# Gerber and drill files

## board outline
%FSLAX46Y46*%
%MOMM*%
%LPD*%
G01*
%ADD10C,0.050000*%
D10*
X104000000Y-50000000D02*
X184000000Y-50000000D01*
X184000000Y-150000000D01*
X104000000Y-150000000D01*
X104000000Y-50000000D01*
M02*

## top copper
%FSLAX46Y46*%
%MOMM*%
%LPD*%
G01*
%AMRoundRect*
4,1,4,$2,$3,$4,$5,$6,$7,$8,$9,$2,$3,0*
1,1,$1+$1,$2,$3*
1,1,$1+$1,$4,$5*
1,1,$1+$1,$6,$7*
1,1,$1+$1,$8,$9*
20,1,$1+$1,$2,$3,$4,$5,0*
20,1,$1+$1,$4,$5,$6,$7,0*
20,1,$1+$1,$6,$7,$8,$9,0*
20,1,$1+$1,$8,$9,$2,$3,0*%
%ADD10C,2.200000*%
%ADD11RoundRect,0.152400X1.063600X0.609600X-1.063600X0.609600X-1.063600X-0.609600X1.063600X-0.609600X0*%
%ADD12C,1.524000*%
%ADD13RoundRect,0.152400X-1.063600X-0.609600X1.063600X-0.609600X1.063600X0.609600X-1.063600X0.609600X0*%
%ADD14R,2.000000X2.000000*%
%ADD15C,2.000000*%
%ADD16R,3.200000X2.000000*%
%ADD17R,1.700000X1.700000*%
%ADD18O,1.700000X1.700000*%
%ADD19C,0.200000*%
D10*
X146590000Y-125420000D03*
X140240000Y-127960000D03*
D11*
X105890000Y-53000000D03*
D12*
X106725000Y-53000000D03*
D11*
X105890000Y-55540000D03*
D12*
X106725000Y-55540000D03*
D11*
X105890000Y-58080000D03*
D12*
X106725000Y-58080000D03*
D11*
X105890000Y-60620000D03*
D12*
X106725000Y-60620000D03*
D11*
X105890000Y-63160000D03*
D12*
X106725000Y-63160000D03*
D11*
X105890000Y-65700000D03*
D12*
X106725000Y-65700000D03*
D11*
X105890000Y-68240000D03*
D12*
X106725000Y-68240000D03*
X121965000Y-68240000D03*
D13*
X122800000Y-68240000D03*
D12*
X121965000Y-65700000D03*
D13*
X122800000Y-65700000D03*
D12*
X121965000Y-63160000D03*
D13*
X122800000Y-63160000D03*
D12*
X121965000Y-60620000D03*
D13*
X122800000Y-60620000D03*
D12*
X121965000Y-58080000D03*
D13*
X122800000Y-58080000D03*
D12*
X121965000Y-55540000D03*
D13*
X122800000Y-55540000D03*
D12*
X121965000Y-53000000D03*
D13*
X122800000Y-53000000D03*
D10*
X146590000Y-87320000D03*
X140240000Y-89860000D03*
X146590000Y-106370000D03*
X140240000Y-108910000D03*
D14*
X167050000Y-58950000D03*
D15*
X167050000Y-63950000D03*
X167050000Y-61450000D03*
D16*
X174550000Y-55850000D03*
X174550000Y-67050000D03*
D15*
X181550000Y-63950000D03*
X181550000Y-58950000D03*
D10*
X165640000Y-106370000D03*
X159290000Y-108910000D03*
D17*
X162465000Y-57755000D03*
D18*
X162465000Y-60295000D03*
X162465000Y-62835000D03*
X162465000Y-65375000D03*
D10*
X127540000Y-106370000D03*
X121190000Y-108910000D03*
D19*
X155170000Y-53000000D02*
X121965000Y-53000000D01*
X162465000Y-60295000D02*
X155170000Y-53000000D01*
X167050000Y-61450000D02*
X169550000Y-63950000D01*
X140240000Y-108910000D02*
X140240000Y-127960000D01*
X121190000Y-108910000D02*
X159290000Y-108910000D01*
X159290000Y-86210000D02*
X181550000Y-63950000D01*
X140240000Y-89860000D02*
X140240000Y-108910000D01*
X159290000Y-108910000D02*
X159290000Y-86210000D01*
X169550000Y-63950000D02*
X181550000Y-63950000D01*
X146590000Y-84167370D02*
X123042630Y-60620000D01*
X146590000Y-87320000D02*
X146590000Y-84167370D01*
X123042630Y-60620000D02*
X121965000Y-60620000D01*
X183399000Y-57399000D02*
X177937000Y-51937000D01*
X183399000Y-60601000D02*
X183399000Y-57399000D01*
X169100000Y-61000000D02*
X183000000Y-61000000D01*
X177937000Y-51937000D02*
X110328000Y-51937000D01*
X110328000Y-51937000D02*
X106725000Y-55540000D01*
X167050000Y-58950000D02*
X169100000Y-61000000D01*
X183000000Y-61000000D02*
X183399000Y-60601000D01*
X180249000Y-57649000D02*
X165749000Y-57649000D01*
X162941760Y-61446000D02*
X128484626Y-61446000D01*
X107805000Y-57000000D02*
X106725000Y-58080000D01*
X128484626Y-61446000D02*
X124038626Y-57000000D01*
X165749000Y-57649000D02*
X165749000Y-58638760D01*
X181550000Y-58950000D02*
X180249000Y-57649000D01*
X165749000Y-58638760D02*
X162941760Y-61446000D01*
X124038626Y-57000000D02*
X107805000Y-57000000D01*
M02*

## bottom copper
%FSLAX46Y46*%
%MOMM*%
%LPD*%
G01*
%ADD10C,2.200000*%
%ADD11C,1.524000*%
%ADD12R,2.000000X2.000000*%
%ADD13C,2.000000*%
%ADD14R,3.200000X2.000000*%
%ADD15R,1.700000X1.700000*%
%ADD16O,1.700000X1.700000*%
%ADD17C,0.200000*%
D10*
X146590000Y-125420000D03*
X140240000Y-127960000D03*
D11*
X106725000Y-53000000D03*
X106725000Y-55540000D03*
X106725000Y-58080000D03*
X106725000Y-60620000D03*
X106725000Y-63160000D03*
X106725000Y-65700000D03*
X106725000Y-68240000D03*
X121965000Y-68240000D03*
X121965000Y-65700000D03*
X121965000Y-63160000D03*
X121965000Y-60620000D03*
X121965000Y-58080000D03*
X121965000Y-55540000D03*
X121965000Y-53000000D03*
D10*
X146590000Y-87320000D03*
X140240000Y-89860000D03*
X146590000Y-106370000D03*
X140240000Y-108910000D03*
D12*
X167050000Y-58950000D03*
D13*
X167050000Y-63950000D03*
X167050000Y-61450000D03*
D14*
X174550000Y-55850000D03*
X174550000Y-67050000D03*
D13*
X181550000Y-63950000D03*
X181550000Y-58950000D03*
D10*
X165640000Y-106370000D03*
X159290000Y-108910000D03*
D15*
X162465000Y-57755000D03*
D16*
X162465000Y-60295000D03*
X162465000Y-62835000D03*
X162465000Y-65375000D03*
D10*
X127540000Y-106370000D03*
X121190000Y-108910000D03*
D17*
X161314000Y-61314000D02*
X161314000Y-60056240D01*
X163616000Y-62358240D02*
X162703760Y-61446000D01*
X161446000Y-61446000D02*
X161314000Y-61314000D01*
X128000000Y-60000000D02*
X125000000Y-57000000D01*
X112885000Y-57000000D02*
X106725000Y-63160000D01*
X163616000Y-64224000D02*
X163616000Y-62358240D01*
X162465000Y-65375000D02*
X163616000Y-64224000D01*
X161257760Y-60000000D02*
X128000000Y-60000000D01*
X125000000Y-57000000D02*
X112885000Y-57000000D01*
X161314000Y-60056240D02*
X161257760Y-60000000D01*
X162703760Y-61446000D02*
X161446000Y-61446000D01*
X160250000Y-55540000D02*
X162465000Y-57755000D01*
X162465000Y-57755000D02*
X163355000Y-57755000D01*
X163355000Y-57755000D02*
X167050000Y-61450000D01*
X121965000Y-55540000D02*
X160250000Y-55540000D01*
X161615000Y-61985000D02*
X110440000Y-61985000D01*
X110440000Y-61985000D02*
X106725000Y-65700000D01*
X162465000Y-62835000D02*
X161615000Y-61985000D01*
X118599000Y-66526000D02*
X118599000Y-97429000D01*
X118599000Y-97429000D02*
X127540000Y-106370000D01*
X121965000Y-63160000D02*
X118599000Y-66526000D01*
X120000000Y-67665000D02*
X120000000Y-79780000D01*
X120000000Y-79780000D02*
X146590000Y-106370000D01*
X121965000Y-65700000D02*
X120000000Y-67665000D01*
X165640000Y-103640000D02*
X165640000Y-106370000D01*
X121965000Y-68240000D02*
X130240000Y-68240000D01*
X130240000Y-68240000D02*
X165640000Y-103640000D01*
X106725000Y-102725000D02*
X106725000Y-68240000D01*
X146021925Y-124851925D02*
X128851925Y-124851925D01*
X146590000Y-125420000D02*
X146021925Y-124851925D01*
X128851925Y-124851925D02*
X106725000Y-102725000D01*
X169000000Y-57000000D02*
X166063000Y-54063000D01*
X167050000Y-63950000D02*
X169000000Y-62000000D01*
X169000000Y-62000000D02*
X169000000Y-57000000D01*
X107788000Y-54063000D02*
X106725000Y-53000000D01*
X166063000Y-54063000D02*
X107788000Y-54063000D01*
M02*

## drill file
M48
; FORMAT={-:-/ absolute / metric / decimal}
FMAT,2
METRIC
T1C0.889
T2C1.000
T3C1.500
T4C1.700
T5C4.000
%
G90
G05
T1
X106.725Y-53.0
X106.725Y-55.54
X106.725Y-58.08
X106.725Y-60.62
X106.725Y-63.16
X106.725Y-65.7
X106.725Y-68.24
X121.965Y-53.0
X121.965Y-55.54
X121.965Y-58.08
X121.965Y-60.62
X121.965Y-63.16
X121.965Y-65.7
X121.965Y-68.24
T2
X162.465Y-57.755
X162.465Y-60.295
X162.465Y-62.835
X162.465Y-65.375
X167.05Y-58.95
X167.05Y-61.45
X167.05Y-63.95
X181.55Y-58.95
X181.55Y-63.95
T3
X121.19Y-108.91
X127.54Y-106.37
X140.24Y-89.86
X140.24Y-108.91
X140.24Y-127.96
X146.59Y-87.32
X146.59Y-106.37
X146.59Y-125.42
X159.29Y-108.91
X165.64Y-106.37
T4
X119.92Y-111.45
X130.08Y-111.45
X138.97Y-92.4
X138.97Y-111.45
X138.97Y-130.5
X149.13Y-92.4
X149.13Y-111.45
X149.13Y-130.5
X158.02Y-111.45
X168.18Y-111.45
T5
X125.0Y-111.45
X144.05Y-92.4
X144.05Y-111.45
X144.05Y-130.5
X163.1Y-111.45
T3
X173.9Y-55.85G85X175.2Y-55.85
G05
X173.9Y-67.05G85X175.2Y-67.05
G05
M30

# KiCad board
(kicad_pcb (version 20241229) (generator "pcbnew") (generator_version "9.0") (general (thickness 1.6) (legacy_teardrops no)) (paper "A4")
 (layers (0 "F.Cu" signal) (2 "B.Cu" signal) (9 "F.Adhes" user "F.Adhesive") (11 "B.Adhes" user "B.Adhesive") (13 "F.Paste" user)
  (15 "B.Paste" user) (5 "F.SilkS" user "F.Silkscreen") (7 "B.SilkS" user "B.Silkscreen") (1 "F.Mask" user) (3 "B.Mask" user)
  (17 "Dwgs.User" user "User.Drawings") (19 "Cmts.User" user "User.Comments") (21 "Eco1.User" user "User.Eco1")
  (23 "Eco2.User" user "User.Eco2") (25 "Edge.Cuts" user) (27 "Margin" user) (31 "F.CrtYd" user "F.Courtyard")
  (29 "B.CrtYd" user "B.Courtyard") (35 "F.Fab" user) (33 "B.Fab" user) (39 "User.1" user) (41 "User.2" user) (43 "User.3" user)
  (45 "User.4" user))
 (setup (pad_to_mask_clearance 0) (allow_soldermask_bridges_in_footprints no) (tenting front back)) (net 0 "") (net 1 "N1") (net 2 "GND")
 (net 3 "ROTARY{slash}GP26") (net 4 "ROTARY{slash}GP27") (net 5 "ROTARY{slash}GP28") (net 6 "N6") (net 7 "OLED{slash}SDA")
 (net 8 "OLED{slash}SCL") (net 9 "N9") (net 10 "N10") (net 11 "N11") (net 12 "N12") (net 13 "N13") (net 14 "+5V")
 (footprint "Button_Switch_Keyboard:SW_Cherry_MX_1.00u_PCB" (layer "F.Cu") (at 146.59 125.42)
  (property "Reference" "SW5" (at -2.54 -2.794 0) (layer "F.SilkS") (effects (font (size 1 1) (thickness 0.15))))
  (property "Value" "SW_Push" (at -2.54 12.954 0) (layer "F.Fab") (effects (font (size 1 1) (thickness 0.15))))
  (pad "" np_thru_hole circle (at -7.62 5.08) (size 1.7 1.7) (drill 1.7) (layers "*.Cu" "*.Mask"))
  (pad "" np_thru_hole circle (at -2.54 5.08) (size 4 4) (drill 4) (layers "*.Cu" "*.Mask"))
  (pad "" np_thru_hole circle (at 2.54 5.08) (size 1.7 1.7) (drill 1.7) (layers "*.Cu" "*.Mask"))
  (pad "1" thru_hole circle (at 0 0) (size 2.2 2.2) (drill 1.5) (layers "*.Cu" "*.Mask") (remove_unused_layers no) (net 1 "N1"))
  (pad "2" thru_hole circle (at -6.35 2.54) (size 2.2 2.2) (drill 1.5) (layers "*.Cu" "*.Mask") (remove_unused_layers no) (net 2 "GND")))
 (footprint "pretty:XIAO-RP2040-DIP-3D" (layer "F.Cu") (at 114.345 60.62)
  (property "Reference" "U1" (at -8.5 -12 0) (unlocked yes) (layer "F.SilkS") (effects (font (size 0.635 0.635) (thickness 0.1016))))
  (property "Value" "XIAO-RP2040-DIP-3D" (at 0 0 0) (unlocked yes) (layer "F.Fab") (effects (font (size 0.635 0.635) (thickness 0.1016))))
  (pad "1" smd roundrect (at -8.455 -7.62 180) (size 2.432 1.524) (layers "F.Cu" "F.Mask") (roundrect_rratio 0.1)
   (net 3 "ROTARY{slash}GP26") (thermal_bridge_angle 45))
  (pad "1" thru_hole circle (at -7.62 -7.62 180) (size 1.524 1.524) (drill 0.889) (layers "*.Cu" "*.Mask") (remove_unused_layers no)
   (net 3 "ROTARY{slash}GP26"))
  (pad "2" smd roundrect (at -8.455 -5.08 180) (size 2.432 1.524) (layers "F.Cu" "F.Mask") (roundrect_rratio 0.1)
   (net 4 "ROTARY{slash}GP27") (thermal_bridge_angle 45))
  (pad "2" thru_hole circle (at -7.62 -5.08 180) (size 1.524 1.524) (drill 0.889) (layers "*.Cu" "*.Mask") (remove_unused_layers no)
   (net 4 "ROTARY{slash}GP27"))
  (pad "3" smd roundrect (at -8.455 -2.54 180) (size 2.432 1.524) (layers "F.Cu" "F.Mask") (roundrect_rratio 0.1)
   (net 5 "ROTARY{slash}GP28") (thermal_bridge_angle 45))
  (pad "3" thru_hole circle (at -7.62 -2.54 180) (size 1.524 1.524) (drill 0.889) (layers "*.Cu" "*.Mask") (remove_unused_layers no)
   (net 5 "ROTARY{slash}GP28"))
  (pad "4" smd roundrect (at -8.455 0 180) (size 2.432 1.524) (layers "F.Cu" "F.Mask") (roundrect_rratio 0.1) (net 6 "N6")
   (thermal_bridge_angle 45))
  (pad "4" thru_hole circle (at -7.62 0 180) (size 1.524 1.524) (drill 0.889) (layers "*.Cu" "*.Mask") (remove_unused_layers no)
   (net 6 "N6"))
  (pad "5" smd roundrect (at -8.455 2.54 180) (size 2.432 1.524) (layers "F.Cu" "F.Mask") (roundrect_rratio 0.1) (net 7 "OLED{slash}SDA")
   (thermal_bridge_angle 45))
  (pad "5" thru_hole circle (at -7.62 2.54 180) (size 1.524 1.524) (drill 0.889) (layers "*.Cu" "*.Mask") (remove_unused_layers no)
   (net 7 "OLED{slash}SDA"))
  (pad "6" smd roundrect (at -8.455 5.08 180) (size 2.432 1.524) (layers "F.Cu" "F.Mask") (roundrect_rratio 0.1) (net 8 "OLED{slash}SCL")
   (thermal_bridge_angle 45))
  (pad "6" thru_hole circle (at -7.62 5.08 180) (size 1.524 1.524) (drill 0.889) (layers "*.Cu" "*.Mask") (remove_unused_layers no)
   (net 8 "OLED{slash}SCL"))
  (pad "7" smd roundrect (at -8.455 7.62 180) (size 2.432 1.524) (layers "F.Cu" "F.Mask") (roundrect_rratio 0.1) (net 1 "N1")
   (thermal_bridge_angle 45))
  (pad "7" thru_hole circle (at -7.62 7.62 180) (size 1.524 1.524) (drill 0.889) (layers "*.Cu" "*.Mask") (remove_unused_layers no)
   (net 1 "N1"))
  (pad "8" thru_hole circle (at 7.62 7.62) (size 1.524 1.524) (drill 0.889) (layers "*.Cu" "*.Mask") (remove_unused_layers no) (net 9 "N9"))
  (pad "8" smd roundrect (at 8.455 7.62) (size 2.432 1.524) (layers "F.Cu" "F.Mask") (roundrect_rratio 0.1) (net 9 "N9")
   (thermal_bridge_angle 45))
  (pad "9" thru_hole circle (at 7.62 5.08) (size 1.524 1.524) (drill 0.889) (layers "*.Cu" "*.Mask") (remove_unused_layers no)
   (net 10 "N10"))
  (pad "9" smd roundrect (at 8.455 5.08) (size 2.432 1.524) (layers "F.Cu" "F.Mask") (roundrect_rratio 0.1) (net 10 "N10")
   (thermal_bridge_angle 45))
  (pad "10" thru_hole circle (at 7.62 2.54) (size 1.524 1.524) (drill 0.889) (layers "*.Cu" "*.Mask") (remove_unused_layers no)
   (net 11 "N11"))
  (pad "10" smd roundrect (at 8.455 2.54) (size 2.432 1.524) (layers "F.Cu" "F.Mask") (roundrect_rratio 0.1) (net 11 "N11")
   (thermal_bridge_angle 45))
  (pad "11" thru_hole circle (at 7.62 0) (size 1.524 1.524) (drill 0.889) (layers "*.Cu" "*.Mask") (remove_unused_layers no) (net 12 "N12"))
  (pad "11" smd roundrect (at 8.455 0) (size 2.432 1.524) (layers "F.Cu" "F.Mask") (roundrect_rratio 0.1) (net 12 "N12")
   (thermal_bridge_angle 45))
  (pad "12" thru_hole circle (at 7.62 -2.54) (size 1.524 1.524) (drill 0.889) (layers "*.Cu" "*.Mask") (remove_unused_layers no)
   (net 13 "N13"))
  (pad "12" smd roundrect (at 8.455 -2.54) (size 2.432 1.524) (layers "F.Cu" "F.Mask") (roundrect_rratio 0.1) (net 13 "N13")
   (thermal_bridge_angle 45))
  (pad "13" thru_hole circle (at 7.62 -5.08) (size 1.524 1.524) (drill 0.889) (layers "*.Cu" "*.Mask") (remove_unused_layers no)
   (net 2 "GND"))
  (pad "13" smd roundrect (at 8.455 -5.08) (size 2.432 1.524) (layers "F.Cu" "F.Mask") (roundrect_rratio 0.1) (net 2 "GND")
   (thermal_bridge_angle 45))
  (pad "14" thru_hole circle (at 7.62 -7.62) (size 1.524 1.524) (drill 0.889) (layers "*.Cu" "*.Mask") (remove_unused_layers no)
   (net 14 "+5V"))
  (pad "14" smd roundrect (at 8.455 -7.62) (size 2.432 1.524) (layers "F.Cu" "F.Mask") (roundrect_rratio 0.1) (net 14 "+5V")
   (thermal_bridge_angle 45)))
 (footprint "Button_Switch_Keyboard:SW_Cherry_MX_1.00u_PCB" (layer "F.Cu") (at 146.59 87.32)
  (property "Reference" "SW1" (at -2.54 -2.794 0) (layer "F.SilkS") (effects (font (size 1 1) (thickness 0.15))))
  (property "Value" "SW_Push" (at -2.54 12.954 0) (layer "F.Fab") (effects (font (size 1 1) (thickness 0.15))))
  (pad "" np_thru_hole circle (at -7.62 5.08) (size 1.7 1.7) (drill 1.7) (layers "*.Cu" "*.Mask"))
  (pad "" np_thru_hole circle (at -2.54 5.08) (size 4 4) (drill 4) (layers "*.Cu" "*.Mask"))
  (pad "" np_thru_hole circle (at 2.54 5.08) (size 1.7 1.7) (drill 1.7) (layers "*.Cu" "*.Mask"))
  (pad "1" thru_hole circle (at 0 0) (size 2.2 2.2) (drill 1.5) (layers "*.Cu" "*.Mask") (remove_unused_layers no) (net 12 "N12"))
  (pad "2" thru_hole circle (at -6.35 2.54) (size 2.2 2.2) (drill 1.5) (layers "*.Cu" "*.Mask") (remove_unused_layers no) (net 2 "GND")))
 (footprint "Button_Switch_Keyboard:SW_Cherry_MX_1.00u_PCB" (layer "F.Cu") (at 146.59 106.37)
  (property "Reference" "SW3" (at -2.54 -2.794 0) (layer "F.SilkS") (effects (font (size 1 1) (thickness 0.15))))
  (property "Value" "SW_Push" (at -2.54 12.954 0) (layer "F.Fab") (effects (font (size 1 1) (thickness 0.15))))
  (pad "" np_thru_hole circle (at -7.62 5.08) (size 1.7 1.7) (drill 1.7) (layers "*.Cu" "*.Mask"))
  (pad "" np_thru_hole circle (at -2.54 5.08) (size 4 4) (drill 4) (layers "*.Cu" "*.Mask"))
  (pad "" np_thru_hole circle (at 2.54 5.08) (size 1.7 1.7) (drill 1.7) (layers "*.Cu" "*.Mask"))
  (pad "1" thru_hole circle (at 0 0) (size 2.2 2.2) (drill 1.5) (layers "*.Cu" "*.Mask") (remove_unused_layers no) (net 10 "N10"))
  (pad "2" thru_hole circle (at -6.35 2.54) (size 2.2 2.2) (drill 1.5) (layers "*.Cu" "*.Mask") (remove_unused_layers no) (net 2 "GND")))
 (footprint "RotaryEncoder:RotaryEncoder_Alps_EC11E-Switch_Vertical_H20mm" (layer "F.Cu") (at 167.05 58.95)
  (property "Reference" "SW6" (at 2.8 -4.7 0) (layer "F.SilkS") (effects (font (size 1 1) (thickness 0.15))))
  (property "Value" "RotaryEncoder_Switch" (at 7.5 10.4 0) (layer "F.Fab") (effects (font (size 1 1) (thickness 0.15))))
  (pad "A" thru_hole rect (at 0 0) (size 2 2) (drill 1) (layers "*.Cu" "*.Mask") (remove_unused_layers no) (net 4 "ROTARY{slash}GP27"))
  (pad "B" thru_hole circle (at 0 5) (size 2 2) (drill 1) (layers "*.Cu" "*.Mask") (remove_unused_layers no) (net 3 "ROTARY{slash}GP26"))
  (pad "C" thru_hole circle (at 0 2.5) (size 2 2) (drill 1) (layers "*.Cu" "*.Mask") (remove_unused_layers no) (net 2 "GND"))
  (pad "MP" thru_hole rect (at 7.5 -3.1) (size 3.2 2) (drill oval 2.8 1.5) (layers "*.Cu" "*.Mask") (remove_unused_layers no))
  (pad "MP" thru_hole rect (at 7.5 8.1) (size 3.2 2) (drill oval 2.8 1.5) (layers "*.Cu" "*.Mask") (remove_unused_layers no))
  (pad "S1" thru_hole circle (at 14.5 5) (size 2 2) (drill 1) (layers "*.Cu" "*.Mask") (remove_unused_layers no) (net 2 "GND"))
  (pad "S2" thru_hole circle (at 14.5 0) (size 2 2) (drill 1) (layers "*.Cu" "*.Mask") (remove_unused_layers no) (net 5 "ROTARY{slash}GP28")))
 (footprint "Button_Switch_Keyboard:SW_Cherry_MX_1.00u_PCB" (layer "F.Cu") (at 165.64 106.37)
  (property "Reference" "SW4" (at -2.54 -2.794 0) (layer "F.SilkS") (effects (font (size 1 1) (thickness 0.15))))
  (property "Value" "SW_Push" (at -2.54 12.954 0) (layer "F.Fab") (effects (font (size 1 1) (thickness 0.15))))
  (pad "" np_thru_hole circle (at -7.62 5.08) (size 1.7 1.7) (drill 1.7) (layers "*.Cu" "*.Mask"))
  (pad "" np_thru_hole circle (at -2.54 5.08) (size 4 4) (drill 4) (layers "*.Cu" "*.Mask"))
  (pad "" np_thru_hole circle (at 2.54 5.08) (size 1.7 1.7) (drill 1.7) (layers "*.Cu" "*.Mask"))
  (pad "1" thru_hole circle (at 0 0) (size 2.2 2.2) (drill 1.5) (layers "*.Cu" "*.Mask") (remove_unused_layers no) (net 9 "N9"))
  (pad "2" thru_hole circle (at -6.35 2.54) (size 2.2 2.2) (drill 1.5) (layers "*.Cu" "*.Mask") (remove_unused_layers no) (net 2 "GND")))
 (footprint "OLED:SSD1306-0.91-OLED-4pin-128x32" (layer "F.Cu") (at 125.965 55.565)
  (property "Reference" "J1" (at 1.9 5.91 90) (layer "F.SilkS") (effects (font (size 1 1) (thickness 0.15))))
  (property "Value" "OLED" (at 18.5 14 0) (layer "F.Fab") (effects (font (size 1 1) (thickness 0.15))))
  (pad "1" thru_hole rect (at 36.5 2.19) (size 1.7 1.7) (drill 1) (layers "*.Cu" "*.Mask") (remove_unused_layers no) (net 2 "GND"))
  (pad "2" thru_hole oval (at 36.5 4.73) (size 1.7 1.7) (drill 1) (layers "*.Cu" "*.Mask") (remove_unused_layers no) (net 14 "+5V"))
  (pad "3" thru_hole oval (at 36.5 7.27) (size 1.7 1.7) (drill 1) (layers "*.Cu" "*.Mask") (remove_unused_layers no)
   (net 8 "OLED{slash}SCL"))
  (pad "4" thru_hole oval (at 36.5 9.81) (size 1.7 1.7) (drill 1) (layers "*.Cu" "*.Mask") (remove_unused_layers no)
   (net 7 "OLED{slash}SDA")))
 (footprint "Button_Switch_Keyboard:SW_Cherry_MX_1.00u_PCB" (layer "F.Cu") (at 127.54 106.37)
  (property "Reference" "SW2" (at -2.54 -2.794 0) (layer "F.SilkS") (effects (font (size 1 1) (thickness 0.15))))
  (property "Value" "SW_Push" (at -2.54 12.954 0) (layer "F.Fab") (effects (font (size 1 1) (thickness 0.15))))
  (pad "" np_thru_hole circle (at -7.62 5.08) (size 1.7 1.7) (drill 1.7) (layers "*.Cu" "*.Mask"))
  (pad "" np_thru_hole circle (at -2.54 5.08) (size 4 4) (drill 4) (layers "*.Cu" "*.Mask"))
  (pad "" np_thru_hole circle (at 2.54 5.08) (size 1.7 1.7) (drill 1.7) (layers "*.Cu" "*.Mask"))
  (pad "1" thru_hole circle (at 0 0) (size 2.2 2.2) (drill 1.5) (layers "*.Cu" "*.Mask") (remove_unused_layers no) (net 11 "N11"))
  (pad "2" thru_hole circle (at -6.35 2.54) (size 2.2 2.2) (drill 1.5) (layers "*.Cu" "*.Mask") (remove_unused_layers no) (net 2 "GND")))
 (gr_rect (start 104 50) (end 184 150) (stroke (width 0.05) (type default)) (fill no) (layer "Edge.Cuts"))
 (segment (start 155.17 53) (end 121.965 53) (width 0.2) (layer "F.Cu") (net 14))
 (segment (start 162.465 60.295) (end 155.17 53) (width 0.2) (layer "F.Cu") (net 14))
 (segment (start 161.314 61.314) (end 161.314 60.05624) (width 0.2) (layer "B.Cu") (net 7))
 (segment (start 163.616 62.35824) (end 162.70376 61.446) (width 0.2) (layer "B.Cu") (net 7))
 (segment (start 161.446 61.446) (end 161.314 61.314) (width 0.2) (layer "B.Cu") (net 7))
 (segment (start 128 60) (end 125 57) (width 0.2) (layer "B.Cu") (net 7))
 (segment (start 112.885 57) (end 106.725 63.16) (width 0.2) (layer "B.Cu") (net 7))
 (segment (start 163.616 64.224) (end 163.616 62.35824) (width 0.2) (layer "B.Cu") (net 7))
 (segment (start 162.465 65.375) (end 163.616 64.224) (width 0.2) (layer "B.Cu") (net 7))
 (segment (start 161.25776 60) (end 128 60) (width 0.2) (layer "B.Cu") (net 7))
 (segment (start 125 57) (end 112.885 57) (width 0.2) (layer "B.Cu") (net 7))
 (segment (start 161.314 60.05624) (end 161.25776 60) (width 0.2) (layer "B.Cu") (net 7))
 (segment (start 162.70376 61.446) (end 161.446 61.446) (width 0.2) (layer "B.Cu") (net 7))
 (segment (start 167.05 61.45) (end 169.55 63.95) (width 0.2) (layer "F.Cu") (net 2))
 (segment (start 140.24 108.91) (end 140.24 127.96) (width 0.2) (layer "F.Cu") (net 2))
 (segment (start 121.19 108.91) (end 159.29 108.91) (width 0.2) (layer "F.Cu") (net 2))
 (segment (start 159.29 86.21) (end 181.55 63.95) (width 0.2) (layer "F.Cu") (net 2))
 (segment (start 140.24 89.86) (end 140.24 108.91) (width 0.2) (layer "F.Cu") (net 2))
 (segment (start 159.29 108.91) (end 159.29 86.21) (width 0.2) (layer "F.Cu") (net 2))
 (segment (start 169.55 63.95) (end 181.55 63.95) (width 0.2) (layer "F.Cu") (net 2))
 (segment (start 160.25 55.54) (end 162.465 57.755) (width 0.2) (layer "B.Cu") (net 2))
 (segment (start 162.465 57.755) (end 163.355 57.755) (width 0.2) (layer "B.Cu") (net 2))
 (segment (start 163.355 57.755) (end 167.05 61.45) (width 0.2) (layer "B.Cu") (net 2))
 (segment (start 121.965 55.54) (end 160.25 55.54) (width 0.2) (layer "B.Cu") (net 2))
 (segment (start 161.615 61.985) (end 110.44 61.985) (width 0.2) (layer "B.Cu") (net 8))
 (segment (start 110.44 61.985) (end 106.725 65.7) (width 0.2) (layer "B.Cu") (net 8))
 (segment (start 162.465 62.835) (end 161.615 61.985) (width 0.2) (layer "B.Cu") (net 8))
 (segment (start 146.59 84.16737) (end 123.04263 60.62) (width 0.2) (layer "F.Cu") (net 12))
 (segment (start 146.59 87.32) (end 146.59 84.16737) (width 0.2) (layer "F.Cu") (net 12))
 (segment (start 123.04263 60.62) (end 121.965 60.62) (width 0.2) (layer "F.Cu") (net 12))
 (segment (start 118.599 66.526) (end 118.599 97.429) (width 0.2) (layer "B.Cu") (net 11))
 (segment (start 118.599 97.429) (end 127.54 106.37) (width 0.2) (layer "B.Cu") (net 11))
 (segment (start 121.965 63.16) (end 118.599 66.526) (width 0.2) (layer "B.Cu") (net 11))
 (segment (start 120 67.665) (end 120 79.78) (width 0.2) (layer "B.Cu") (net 10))
 (segment (start 120 79.78) (end 146.59 106.37) (width 0.2) (layer "B.Cu") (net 10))
 (segment (start 121.965 65.7) (end 120 67.665) (width 0.2) (layer "B.Cu") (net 10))
 (segment (start 165.64 103.64) (end 165.64 106.37) (width 0.2) (layer "B.Cu") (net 9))
 (segment (start 121.965 68.24) (end 130.24 68.24) (width 0.2) (layer "B.Cu") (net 9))
 (segment (start 130.24 68.24) (end 165.64 103.64) (width 0.2) (layer "B.Cu") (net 9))
 (segment (start 106.725 102.725) (end 106.725 68.24) (width 0.2) (layer "B.Cu") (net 1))
 (segment (start 146.021925 124.851925) (end 128.851925 124.851925) (width 0.2) (layer "B.Cu") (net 1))
 (segment (start 146.59 125.42) (end 146.021925 124.851925) (width 0.2) (layer "B.Cu") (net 1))
 (segment (start 128.851925 124.851925) (end 106.725 102.725) (width 0.2) (layer "B.Cu") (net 1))
 (segment (start 183.399 57.399) (end 177.937 51.937) (width 0.2) (layer "F.Cu") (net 4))
 (segment (start 183.399 60.601) (end 183.399 57.399) (width 0.2) (layer "F.Cu") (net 4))
 (segment (start 169.1 61) (end 183 61) (width 0.2) (layer "F.Cu") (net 4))
 (segment (start 177.937 51.937) (end 110.328 51.937) (width 0.2) (layer "F.Cu") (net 4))
 (segment (start 110.328 51.937) (end 106.725 55.54) (width 0.2) (layer "F.Cu") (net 4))
 (segment (start 167.05 58.95) (end 169.1 61) (width 0.2) (layer "F.Cu") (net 4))
 (segment (start 183 61) (end 183.399 60.601) (width 0.2) (layer "F.Cu") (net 4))
 (segment (start 180.249 57.649) (end 165.749 57.649) (width 0.2) (layer "F.Cu") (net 5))
 (segment (start 162.94176 61.446) (end 128.484626 61.446) (width 0.2) (layer "F.Cu") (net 5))
 (segment (start 107.805 57) (end 106.725 58.08) (width 0.2) (layer "F.Cu") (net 5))
 (segment (start 128.484626 61.446) (end 124.038626 57) (width 0.2) (layer "F.Cu") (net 5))
 (segment (start 165.749 57.649) (end 165.749 58.63876) (width 0.2) (layer "F.Cu") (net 5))
 (segment (start 181.55 58.95) (end 180.249 57.649) (width 0.2) (layer "F.Cu") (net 5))
 (segment (start 165.749 58.63876) (end 162.94176 61.446) (width 0.2) (layer "F.Cu") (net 5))
 (segment (start 124.038626 57) (end 107.805 57) (width 0.2) (layer "F.Cu") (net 5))
 (segment (start 169 57) (end 166.063 54.063) (width 0.2) (layer "B.Cu") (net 3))
 (segment (start 167.05 63.95) (end 169 62) (width 0.2) (layer "B.Cu") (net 3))
 (segment (start 169 62) (end 169 57) (width 0.2) (layer "B.Cu") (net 3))
 (segment (start 107.788 54.063) (end 106.725 53) (width 0.2) (layer "B.Cu") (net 3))
 (segment (start 166.063 54.063) (end 107.788 54.063) (width 0.2) (layer "B.Cu") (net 3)))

